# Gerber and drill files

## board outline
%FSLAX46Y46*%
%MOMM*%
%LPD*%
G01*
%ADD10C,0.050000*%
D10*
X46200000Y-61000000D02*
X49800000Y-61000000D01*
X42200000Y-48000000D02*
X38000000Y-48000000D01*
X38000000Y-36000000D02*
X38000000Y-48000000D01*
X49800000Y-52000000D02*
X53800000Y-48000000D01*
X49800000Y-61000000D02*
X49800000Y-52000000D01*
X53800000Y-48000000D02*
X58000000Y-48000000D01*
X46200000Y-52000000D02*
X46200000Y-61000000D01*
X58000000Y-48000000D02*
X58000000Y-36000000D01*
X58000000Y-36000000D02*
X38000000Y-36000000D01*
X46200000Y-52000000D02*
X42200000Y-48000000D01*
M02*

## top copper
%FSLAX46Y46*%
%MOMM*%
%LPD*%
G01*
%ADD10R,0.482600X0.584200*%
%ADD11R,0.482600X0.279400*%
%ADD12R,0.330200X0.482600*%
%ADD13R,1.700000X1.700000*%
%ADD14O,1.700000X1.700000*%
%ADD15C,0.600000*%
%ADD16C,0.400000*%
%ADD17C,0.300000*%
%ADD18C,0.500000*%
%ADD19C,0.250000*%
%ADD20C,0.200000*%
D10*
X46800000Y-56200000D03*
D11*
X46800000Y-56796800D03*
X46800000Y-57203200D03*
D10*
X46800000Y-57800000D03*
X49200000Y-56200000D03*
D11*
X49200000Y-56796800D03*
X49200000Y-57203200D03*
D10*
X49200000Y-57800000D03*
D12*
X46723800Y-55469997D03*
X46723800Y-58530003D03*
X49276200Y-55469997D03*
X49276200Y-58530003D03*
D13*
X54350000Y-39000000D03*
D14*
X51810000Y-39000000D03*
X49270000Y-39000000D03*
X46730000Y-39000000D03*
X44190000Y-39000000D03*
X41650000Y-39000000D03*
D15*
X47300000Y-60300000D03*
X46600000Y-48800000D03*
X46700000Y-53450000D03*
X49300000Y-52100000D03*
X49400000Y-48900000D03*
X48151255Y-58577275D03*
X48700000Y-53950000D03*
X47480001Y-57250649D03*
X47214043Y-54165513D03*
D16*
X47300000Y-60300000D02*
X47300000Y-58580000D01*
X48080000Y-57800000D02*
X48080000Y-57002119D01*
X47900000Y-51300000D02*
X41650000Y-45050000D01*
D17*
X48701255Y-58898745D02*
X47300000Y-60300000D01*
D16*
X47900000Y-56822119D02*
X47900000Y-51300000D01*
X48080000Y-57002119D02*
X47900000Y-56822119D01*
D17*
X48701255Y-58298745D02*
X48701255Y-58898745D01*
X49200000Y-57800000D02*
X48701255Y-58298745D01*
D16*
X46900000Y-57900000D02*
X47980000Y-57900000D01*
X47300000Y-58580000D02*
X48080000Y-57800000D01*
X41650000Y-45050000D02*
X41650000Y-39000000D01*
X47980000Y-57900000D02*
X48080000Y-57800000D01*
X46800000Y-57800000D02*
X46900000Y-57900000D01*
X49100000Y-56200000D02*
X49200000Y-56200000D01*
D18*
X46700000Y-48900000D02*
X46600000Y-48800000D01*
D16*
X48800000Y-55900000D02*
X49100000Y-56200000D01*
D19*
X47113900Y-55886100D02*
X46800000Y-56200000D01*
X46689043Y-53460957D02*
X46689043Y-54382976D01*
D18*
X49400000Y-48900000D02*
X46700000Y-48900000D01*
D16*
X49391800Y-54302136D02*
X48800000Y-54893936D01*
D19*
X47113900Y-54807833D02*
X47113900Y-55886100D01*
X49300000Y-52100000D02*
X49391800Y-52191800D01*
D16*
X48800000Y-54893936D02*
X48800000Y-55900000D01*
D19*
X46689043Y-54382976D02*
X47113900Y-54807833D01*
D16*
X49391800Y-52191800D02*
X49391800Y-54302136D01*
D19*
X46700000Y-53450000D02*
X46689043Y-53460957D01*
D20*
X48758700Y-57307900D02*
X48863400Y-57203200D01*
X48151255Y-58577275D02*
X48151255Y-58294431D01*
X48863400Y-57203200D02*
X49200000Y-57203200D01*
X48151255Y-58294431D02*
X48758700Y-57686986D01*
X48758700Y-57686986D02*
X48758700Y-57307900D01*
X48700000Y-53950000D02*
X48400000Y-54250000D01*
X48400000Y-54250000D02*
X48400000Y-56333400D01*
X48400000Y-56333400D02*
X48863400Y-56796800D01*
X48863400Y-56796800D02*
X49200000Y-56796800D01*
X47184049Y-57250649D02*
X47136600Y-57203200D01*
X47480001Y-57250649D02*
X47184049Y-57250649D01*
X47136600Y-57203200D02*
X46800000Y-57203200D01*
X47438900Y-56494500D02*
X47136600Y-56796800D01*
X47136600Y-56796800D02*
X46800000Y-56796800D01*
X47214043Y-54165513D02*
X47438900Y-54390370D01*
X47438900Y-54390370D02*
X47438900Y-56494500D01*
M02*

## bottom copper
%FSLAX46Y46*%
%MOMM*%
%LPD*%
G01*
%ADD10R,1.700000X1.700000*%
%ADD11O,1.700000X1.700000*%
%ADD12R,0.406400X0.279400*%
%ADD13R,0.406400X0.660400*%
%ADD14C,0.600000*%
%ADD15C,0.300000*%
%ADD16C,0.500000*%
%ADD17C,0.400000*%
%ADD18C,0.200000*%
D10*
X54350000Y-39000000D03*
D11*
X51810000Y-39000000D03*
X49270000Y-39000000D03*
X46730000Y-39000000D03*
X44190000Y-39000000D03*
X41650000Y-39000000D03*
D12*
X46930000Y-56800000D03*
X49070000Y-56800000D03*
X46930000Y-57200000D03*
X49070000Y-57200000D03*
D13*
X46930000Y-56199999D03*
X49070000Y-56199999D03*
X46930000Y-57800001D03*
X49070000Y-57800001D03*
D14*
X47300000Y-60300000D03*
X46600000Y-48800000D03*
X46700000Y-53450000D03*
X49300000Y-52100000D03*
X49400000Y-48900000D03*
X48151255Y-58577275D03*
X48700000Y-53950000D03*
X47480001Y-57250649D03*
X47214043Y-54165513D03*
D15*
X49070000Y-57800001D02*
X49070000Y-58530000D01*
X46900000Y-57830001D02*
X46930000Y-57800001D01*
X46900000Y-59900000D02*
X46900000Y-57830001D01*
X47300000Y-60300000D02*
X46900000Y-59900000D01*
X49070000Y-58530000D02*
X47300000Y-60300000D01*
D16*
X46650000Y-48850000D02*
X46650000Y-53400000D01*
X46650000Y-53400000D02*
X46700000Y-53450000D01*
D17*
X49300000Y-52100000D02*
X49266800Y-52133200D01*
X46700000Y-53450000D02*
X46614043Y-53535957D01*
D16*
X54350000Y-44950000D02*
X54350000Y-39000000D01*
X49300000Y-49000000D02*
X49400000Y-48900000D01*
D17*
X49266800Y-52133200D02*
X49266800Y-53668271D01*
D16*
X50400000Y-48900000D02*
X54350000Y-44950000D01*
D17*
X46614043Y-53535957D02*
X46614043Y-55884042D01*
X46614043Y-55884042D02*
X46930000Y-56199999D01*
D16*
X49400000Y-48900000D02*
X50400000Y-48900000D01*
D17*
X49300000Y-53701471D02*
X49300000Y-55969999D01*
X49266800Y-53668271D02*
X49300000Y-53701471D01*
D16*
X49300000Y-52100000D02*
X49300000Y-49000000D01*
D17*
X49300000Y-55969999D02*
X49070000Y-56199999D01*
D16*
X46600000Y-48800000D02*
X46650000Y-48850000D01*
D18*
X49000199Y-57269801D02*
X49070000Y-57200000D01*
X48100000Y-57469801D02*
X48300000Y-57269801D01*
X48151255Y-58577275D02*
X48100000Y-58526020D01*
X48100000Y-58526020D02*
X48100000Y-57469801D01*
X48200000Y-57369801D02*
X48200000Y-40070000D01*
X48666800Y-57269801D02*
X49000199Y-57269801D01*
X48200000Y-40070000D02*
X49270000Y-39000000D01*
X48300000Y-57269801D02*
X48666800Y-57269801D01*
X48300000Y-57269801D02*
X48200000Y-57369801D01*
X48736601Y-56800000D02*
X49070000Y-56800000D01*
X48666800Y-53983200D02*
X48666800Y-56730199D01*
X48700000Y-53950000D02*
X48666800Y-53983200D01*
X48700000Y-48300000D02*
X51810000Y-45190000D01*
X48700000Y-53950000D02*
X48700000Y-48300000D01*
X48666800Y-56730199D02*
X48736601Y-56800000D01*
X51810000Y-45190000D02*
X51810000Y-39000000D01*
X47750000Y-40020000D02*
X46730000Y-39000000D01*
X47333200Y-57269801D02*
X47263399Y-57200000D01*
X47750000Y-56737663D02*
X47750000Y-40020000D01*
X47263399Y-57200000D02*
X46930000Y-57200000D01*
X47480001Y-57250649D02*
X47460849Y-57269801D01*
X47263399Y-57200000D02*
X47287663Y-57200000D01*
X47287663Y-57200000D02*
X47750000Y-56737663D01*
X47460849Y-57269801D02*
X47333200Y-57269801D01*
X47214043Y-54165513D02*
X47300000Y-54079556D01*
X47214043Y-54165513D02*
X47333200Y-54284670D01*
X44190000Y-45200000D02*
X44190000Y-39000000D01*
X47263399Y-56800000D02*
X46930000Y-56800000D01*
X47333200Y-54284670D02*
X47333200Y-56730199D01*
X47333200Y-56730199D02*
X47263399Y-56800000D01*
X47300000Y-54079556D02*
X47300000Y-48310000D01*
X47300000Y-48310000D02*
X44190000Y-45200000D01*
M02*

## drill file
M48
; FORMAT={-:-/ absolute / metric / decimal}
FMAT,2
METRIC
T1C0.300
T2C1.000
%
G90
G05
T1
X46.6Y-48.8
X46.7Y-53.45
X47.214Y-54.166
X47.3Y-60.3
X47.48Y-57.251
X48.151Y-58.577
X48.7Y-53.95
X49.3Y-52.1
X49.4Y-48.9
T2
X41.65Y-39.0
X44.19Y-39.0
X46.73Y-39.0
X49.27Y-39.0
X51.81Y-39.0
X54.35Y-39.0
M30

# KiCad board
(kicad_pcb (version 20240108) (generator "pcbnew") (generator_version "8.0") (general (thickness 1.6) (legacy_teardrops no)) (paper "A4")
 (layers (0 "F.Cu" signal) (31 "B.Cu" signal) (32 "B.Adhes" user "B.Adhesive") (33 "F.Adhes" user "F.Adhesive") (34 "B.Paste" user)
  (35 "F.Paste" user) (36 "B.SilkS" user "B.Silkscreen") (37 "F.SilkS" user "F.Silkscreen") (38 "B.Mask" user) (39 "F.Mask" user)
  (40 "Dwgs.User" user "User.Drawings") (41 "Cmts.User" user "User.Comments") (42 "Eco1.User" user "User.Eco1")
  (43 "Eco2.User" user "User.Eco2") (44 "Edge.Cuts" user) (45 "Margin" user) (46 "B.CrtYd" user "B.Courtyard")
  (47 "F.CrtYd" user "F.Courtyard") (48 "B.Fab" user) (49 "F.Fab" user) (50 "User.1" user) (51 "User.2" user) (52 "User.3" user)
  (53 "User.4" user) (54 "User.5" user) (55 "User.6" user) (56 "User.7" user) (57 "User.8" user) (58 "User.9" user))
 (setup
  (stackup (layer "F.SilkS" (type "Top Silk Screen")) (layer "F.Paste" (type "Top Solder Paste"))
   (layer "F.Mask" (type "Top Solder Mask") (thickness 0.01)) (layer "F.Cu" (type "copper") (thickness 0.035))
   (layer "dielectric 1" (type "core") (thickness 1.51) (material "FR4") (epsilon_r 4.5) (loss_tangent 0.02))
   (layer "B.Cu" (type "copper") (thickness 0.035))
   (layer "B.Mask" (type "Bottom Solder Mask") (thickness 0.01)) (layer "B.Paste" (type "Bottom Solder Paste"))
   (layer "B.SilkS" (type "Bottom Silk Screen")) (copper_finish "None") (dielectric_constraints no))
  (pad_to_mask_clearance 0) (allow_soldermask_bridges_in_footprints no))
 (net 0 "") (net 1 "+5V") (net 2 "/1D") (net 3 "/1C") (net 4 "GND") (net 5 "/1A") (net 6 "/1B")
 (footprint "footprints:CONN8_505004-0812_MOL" (layer "F.Cu") (at 48 57 90)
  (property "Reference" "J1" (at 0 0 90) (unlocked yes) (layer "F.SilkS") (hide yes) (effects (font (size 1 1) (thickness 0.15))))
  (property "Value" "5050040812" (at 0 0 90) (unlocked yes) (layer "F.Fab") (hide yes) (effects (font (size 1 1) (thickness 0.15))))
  (pad "1" smd rect (at 0.8 -1.2 90) (size 0.5842 0.4826) (layers "F.Cu" "F.Paste" "F.Mask") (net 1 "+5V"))
  (pad "2" smd rect (at 0.2032 -1.2 90) (size 0.2794 0.4826) (layers "F.Cu" "F.Paste" "F.Mask") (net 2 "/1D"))
  (pad "3" smd rect (at -0.2032 -1.2 90) (size 0.2794 0.4826) (layers "F.Cu" "F.Paste" "F.Mask") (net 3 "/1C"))
  (pad "4" smd rect (at -0.8 -1.2 90) (size 0.5842 0.4826) (layers "F.Cu" "F.Paste" "F.Mask") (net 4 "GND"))
  (pad "5" smd rect (at 0.8 1.2 90) (size 0.5842 0.4826) (layers "F.Cu" "F.Paste" "F.Mask") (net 1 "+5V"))
  (pad "6" smd rect (at 0.2032 1.2 90) (size 0.2794 0.4826) (layers "F.Cu" "F.Paste" "F.Mask") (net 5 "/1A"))
  (pad "7" smd rect (at -0.2032 1.2 90) (size 0.2794 0.4826) (layers "F.Cu" "F.Paste" "F.Mask") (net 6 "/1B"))
  (pad "8" smd rect (at -0.8 1.2 90) (size 0.5842 0.4826) (layers "F.Cu" "F.Paste" "F.Mask") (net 4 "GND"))
  (pad "9" smd rect (at 1.530003 -1.2762 90) (size 0.4826 0.3302) (layers "F.Cu" "F.Paste" "F.Mask"))
  (pad "10" smd rect (at -1.530003 -1.2762 90) (size 0.4826 0.3302) (layers "F.Cu" "F.Paste" "F.Mask"))
  (pad "11" smd rect (at 1.530003 1.2762 90) (size 0.4826 0.3302) (layers "F.Cu" "F.Paste" "F.Mask"))
  (pad "12" smd rect (at -1.530003 1.2762 90) (size 0.4826 0.3302) (layers "F.Cu" "F.Paste" "F.Mask")))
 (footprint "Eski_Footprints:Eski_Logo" (layer "F.Cu") (at 48 47.65)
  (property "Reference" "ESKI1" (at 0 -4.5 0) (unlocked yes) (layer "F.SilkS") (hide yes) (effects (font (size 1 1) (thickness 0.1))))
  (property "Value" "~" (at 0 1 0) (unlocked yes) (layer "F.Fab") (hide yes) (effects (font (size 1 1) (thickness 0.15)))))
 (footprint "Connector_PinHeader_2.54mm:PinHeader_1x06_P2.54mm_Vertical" (layer "F.Cu") (at 54.35 39 -90)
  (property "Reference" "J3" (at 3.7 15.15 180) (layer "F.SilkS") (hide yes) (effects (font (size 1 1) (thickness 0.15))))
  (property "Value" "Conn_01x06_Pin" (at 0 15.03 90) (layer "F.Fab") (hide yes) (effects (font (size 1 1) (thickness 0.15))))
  (pad "1" thru_hole rect (at 0 0 270) (size 1.7 1.7) (drill 1) (layers "*.Cu" "*.Mask") (remove_unused_layers no) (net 1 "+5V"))
  (pad "2" thru_hole oval (at 0 2.54 270) (size 1.7 1.7) (drill 1) (layers "*.Cu" "*.Mask") (remove_unused_layers no) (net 5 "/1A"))
  (pad "3" thru_hole oval (at 0 5.08 270) (size 1.7 1.7) (drill 1) (layers "*.Cu" "*.Mask") (remove_unused_layers no) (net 6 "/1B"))
  (pad "4" thru_hole oval (at 0 7.62 270) (size 1.7 1.7) (drill 1) (layers "*.Cu" "*.Mask") (remove_unused_layers no) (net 3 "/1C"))
  (pad "5" thru_hole oval (at 0 10.16 270) (size 1.7 1.7) (drill 1) (layers "*.Cu" "*.Mask") (remove_unused_layers no) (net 2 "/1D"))
  (pad "6" thru_hole oval (at 0 12.7 270) (size 1.7 1.7) (drill 1) (layers "*.Cu" "*.Mask") (remove_unused_layers no) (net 4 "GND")))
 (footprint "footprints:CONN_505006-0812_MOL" (layer "B.Cu") (at 48 57 -90)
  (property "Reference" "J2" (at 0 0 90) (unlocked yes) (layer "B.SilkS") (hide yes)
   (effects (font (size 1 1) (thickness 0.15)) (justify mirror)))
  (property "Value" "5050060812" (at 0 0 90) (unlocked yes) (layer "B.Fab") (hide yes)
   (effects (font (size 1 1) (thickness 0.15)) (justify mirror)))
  (pad "1" smd rect (at -0.2 1.07 270) (size 0.2794 0.4064) (layers "B.Cu" "B.Paste" "B.Mask") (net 2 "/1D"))
  (pad "2" smd rect (at -0.2 -1.07 270) (size 0.2794 0.4064) (layers "B.Cu" "B.Paste" "B.Mask") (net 5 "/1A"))
  (pad "3" smd rect (at 0.2 1.07 270) (size 0.2794 0.4064) (layers "B.Cu" "B.Paste" "B.Mask") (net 3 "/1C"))
  (pad "4" smd rect (at 0.2 -1.07 270) (size 0.2794 0.4064) (layers "B.Cu" "B.Paste" "B.Mask") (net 6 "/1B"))
  (pad "P1" smd rect (at -0.800001 1.07 270) (size 0.6604 0.4064) (layers "B.Cu" "B.Paste" "B.Mask") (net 1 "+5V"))
  (pad "P2" smd rect (at -0.800001 -1.07 270) (size 0.6604 0.4064) (layers "B.Cu" "B.Paste" "B.Mask") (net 1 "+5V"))
  (pad "P3" smd rect (at 0.800001 1.07 270) (size 0.6604 0.4064) (layers "B.Cu" "B.Paste" "B.Mask") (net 4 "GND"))
  (pad "P4" smd rect (at 0.800001 -1.07 270) (size 0.6604 0.4064) (layers "B.Cu" "B.Paste" "B.Mask") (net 4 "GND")))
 (gr_line (start 46.2 61) (end 49.8 61) (stroke (width 0.05) (type default)) (layer "Edge.Cuts"))
 (gr_line (start 42.2 48) (end 38 48) (stroke (width 0.05) (type default)) (layer "Edge.Cuts"))
 (gr_line (start 38 36) (end 38 48) (stroke (width 0.05) (type default)) (layer "Edge.Cuts"))
 (gr_line (start 49.8 52) (end 53.8 48) (stroke (width 0.05) (type default)) (layer "Edge.Cuts"))
 (gr_line (start 49.8 61) (end 49.8 52) (stroke (width 0.05) (type default)) (layer "Edge.Cuts"))
 (gr_line (start 53.8 48) (end 58 48) (stroke (width 0.05) (type default)) (layer "Edge.Cuts"))
 (gr_line (start 46.2 52) (end 46.2 61) (stroke (width 0.05) (type default)) (layer "Edge.Cuts"))
 (gr_line (start 58 48) (end 58 36) (stroke (width 0.05) (type default)) (layer "Edge.Cuts"))
 (gr_line (start 58 36) (end 38 36) (stroke (width 0.05) (type default)) (layer "Edge.Cuts"))
 (gr_line (start 46.2 52) (end 42.2 48) (stroke (width 0.05) (type default)) (layer "Edge.Cuts"))
 (segment (start 47.3 60.3) (end 47.3 58.58) (width 0.4) (layer "F.Cu") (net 4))
 (segment (start 48.08 57.8) (end 48.08 57.002119) (width 0.4) (layer "F.Cu") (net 4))
 (segment (start 47.9 51.3) (end 41.65 45.05) (width 0.4) (layer "F.Cu") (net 4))
 (segment (start 48.701255 58.898745) (end 47.3 60.3) (width 0.3) (layer "F.Cu") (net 4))
 (segment (start 47.9 56.822119) (end 47.9 51.3) (width 0.4) (layer "F.Cu") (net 4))
 (segment (start 48.08 57.002119) (end 47.9 56.822119) (width 0.4) (layer "F.Cu") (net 4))
 (segment (start 48.701255 58.298745) (end 48.701255 58.898745) (width 0.3) (layer "F.Cu") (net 4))
 (segment (start 49.2 57.8) (end 48.701255 58.298745) (width 0.3) (layer "F.Cu") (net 4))
 (segment (start 46.9 57.9) (end 47.98 57.9) (width 0.4) (layer "F.Cu") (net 4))
 (segment (start 47.3 58.58) (end 48.08 57.8) (width 0.4) (layer "F.Cu") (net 4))
 (segment (start 41.65 45.05) (end 41.65 39) (width 0.4) (layer "F.Cu") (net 4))
 (segment (start 47.98 57.9) (end 48.08 57.8) (width 0.4) (layer "F.Cu") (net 4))
 (segment (start 46.8 57.8) (end 46.9 57.9) (width 0.4) (layer "F.Cu") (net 4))
 (via (at 47.3 60.3) (size 0.6) (drill 0.3) (layers "F.Cu" "B.Cu") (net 4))
 (segment (start 49.07 57.800001) (end 49.07 58.53) (width 0.3) (layer "B.Cu") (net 4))
 (segment (start 46.9 57.830001) (end 46.93 57.800001) (width 0.3) (layer "B.Cu") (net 4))
 (segment (start 46.9 59.9) (end 46.9 57.830001) (width 0.3) (layer "B.Cu") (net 4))
 (segment (start 47.3 60.3) (end 46.9 59.9) (width 0.3) (layer "B.Cu") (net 4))
 (segment (start 49.07 58.53) (end 47.3 60.3) (width 0.3) (layer "B.Cu") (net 4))
 (segment (start 49.1 56.2) (end 49.2 56.2) (width 0.4) (layer "F.Cu") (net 1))
 (segment (start 46.7 48.9) (end 46.6 48.8) (width 0.5) (layer "F.Cu") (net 1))
 (segment (start 48.8 55.9) (end 49.1 56.2) (width 0.4) (layer "F.Cu") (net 1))
 (segment (start 47.1139 55.8861) (end 46.8 56.2) (width 0.25) (layer "F.Cu") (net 1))
 (segment (start 46.689043 53.460957) (end 46.689043 54.382976) (width 0.25) (layer "F.Cu") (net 1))
 (segment (start 49.4 48.9) (end 46.7 48.9) (width 0.5) (layer "F.Cu") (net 1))
 (segment (start 49.3918 54.302136) (end 48.8 54.893936) (width 0.4) (layer "F.Cu") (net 1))
 (segment (start 47.1139 54.807833) (end 47.1139 55.8861) (width 0.25) (layer "F.Cu") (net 1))
 (segment (start 49.3 52.1) (end 49.3918 52.1918) (width 0.25) (layer "F.Cu") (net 1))
 (segment (start 48.8 54.893936) (end 48.8 55.9) (width 0.4) (layer "F.Cu") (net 1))
 (segment (start 46.689043 54.382976) (end 47.1139 54.807833) (width 0.25) (layer "F.Cu") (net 1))
 (segment (start 49.3918 52.1918) (end 49.3918 54.302136) (width 0.4) (layer "F.Cu") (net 1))
 (segment (start 46.7 53.45) (end 46.689043 53.460957) (width 0.25) (layer "F.Cu") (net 1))
 (via (at 46.6 48.8) (size 0.6) (drill 0.3) (layers "F.Cu" "B.Cu") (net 1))
 (via (at 46.7 53.45) (size 0.6) (drill 0.3) (layers "F.Cu" "B.Cu") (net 1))
 (via (at 49.3 52.1) (size 0.6) (drill 0.3) (layers "F.Cu" "B.Cu") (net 1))
 (via (at 49.4 48.9) (size 0.6) (drill 0.3) (layers "F.Cu" "B.Cu") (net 1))
 (segment (start 46.65 48.85) (end 46.65 53.4) (width 0.5) (layer "B.Cu") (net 1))
 (segment (start 46.65 53.4) (end 46.7 53.45) (width 0.5) (layer "B.Cu") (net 1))
 (segment (start 49.3 52.1) (end 49.2668 52.1332) (width 0.4) (layer "B.Cu") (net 1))
 (segment (start 46.7 53.45) (end 46.614043 53.535957) (width 0.4) (layer "B.Cu") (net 1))
 (segment (start 54.35 44.95) (end 54.35 39) (width 0.5) (layer "B.Cu") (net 1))
 (segment (start 49.3 49) (end 49.4 48.9) (width 0.5) (layer "B.Cu") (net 1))
 (segment (start 49.2668 52.1332) (end 49.2668 53.668271) (width 0.4) (layer "B.Cu") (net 1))
 (segment (start 50.4 48.9) (end 54.35 44.95) (width 0.5) (layer "B.Cu") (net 1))
 (segment (start 46.614043 53.535957) (end 46.614043 55.884042) (width 0.4) (layer "B.Cu") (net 1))
 (segment (start 46.614043 55.884042) (end 46.93 56.199999) (width 0.4) (layer "B.Cu") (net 1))
 (segment (start 49.4 48.9) (end 50.4 48.9) (width 0.5) (layer "B.Cu") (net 1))
 (segment (start 49.3 53.701471) (end 49.3 55.969999) (width 0.4) (layer "B.Cu") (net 1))
 (segment (start 49.2668 53.668271) (end 49.3 53.701471) (width 0.4) (layer "B.Cu") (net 1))
 (segment (start 49.3 52.1) (end 49.3 49) (width 0.5) (layer "B.Cu") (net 1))
 (segment (start 49.3 55.969999) (end 49.07 56.199999) (width 0.4) (layer "B.Cu") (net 1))
 (segment (start 46.6 48.8) (end 46.65 48.85) (width 0.5) (layer "B.Cu") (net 1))
 (segment (start 48.7587 57.3079) (end 48.8634 57.2032) (width 0.2) (layer "F.Cu") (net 6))
 (segment (start 48.151255 58.577275) (end 48.151255 58.294431) (width 0.2) (layer "F.Cu") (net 6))
 (segment (start 48.8634 57.2032) (end 49.2 57.2032) (width 0.2) (layer "F.Cu") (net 6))
 (segment (start 48.151255 58.294431) (end 48.7587 57.686986) (width 0.2) (layer "F.Cu") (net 6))
 (segment (start 48.7587 57.686986) (end 48.7587 57.3079) (width 0.2) (layer "F.Cu") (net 6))
 (via (at 48.151255 58.577275) (size 0.6) (drill 0.3) (layers "F.Cu" "B.Cu") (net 6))
 (segment (start 49.000199 57.269801) (end 49.07 57.2) (width 0.2) (layer "B.Cu") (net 6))
 (segment (start 48.1 57.469801) (end 48.3 57.269801) (width 0.2) (layer "B.Cu") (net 6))
 (segment (start 48.151255 58.577275) (end 48.1 58.52602) (width 0.2) (layer "B.Cu") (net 6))
 (segment (start 48.1 58.52602) (end 48.1 57.469801) (width 0.2) (layer "B.Cu") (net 6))
 (segment (start 48.2 57.369801) (end 48.2 40.07) (width 0.2) (layer "B.Cu") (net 6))
 (segment (start 48.6668 57.269801) (end 49.000199 57.269801) (width 0.2) (layer "B.Cu") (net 6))
 (segment (start 48.2 40.07) (end 49.27 39) (width 0.2) (layer "B.Cu") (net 6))
 (segment (start 48.3 57.269801) (end 48.6668 57.269801) (width 0.2) (layer "B.Cu") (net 6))
 (segment (start 48.3 57.269801) (end 48.2 57.369801) (width 0.2) (layer "B.Cu") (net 6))
 (segment (start 48.7 53.95) (end 48.4 54.25) (width 0.2) (layer "F.Cu") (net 5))
 (segment (start 48.4 54.25) (end 48.4 56.3334) (width 0.2) (layer "F.Cu") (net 5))
 (segment (start 48.4 56.3334) (end 48.8634 56.7968) (width 0.2) (layer "F.Cu") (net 5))
 (segment (start 48.8634 56.7968) (end 49.2 56.7968) (width 0.2) (layer "F.Cu") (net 5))
 (via (at 48.7 53.95) (size 0.6) (drill 0.3) (layers "F.Cu" "B.Cu") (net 5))
 (segment (start 48.736601 56.8) (end 49.07 56.8) (width 0.2) (layer "B.Cu") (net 5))
 (segment (start 48.6668 53.9832) (end 48.6668 56.730199) (width 0.2) (layer "B.Cu") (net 5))
 (segment (start 48.7 53.95) (end 48.6668 53.9832) (width 0.2) (layer "B.Cu") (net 5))
 (segment (start 48.7 48.3) (end 51.81 45.19) (width 0.2) (layer "B.Cu") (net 5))
 (segment (start 48.7 53.95) (end 48.7 48.3) (width 0.2) (layer "B.Cu") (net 5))
 (segment (start 48.6668 56.730199) (end 48.736601 56.8) (width 0.2) (layer "B.Cu") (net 5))
 (segment (start 51.81 45.19) (end 51.81 39) (width 0.2) (layer "B.Cu") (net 5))
 (segment (start 47.184049 57.250649) (end 47.1366 57.2032) (width 0.2) (layer "F.Cu") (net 3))
 (segment (start 47.480001 57.250649) (end 47.184049 57.250649) (width 0.2) (layer "F.Cu") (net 3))
 (segment (start 47.1366 57.2032) (end 46.8 57.2032) (width 0.2) (layer "F.Cu") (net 3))
 (via (at 47.480001 57.250649) (size 0.6) (drill 0.3) (layers "F.Cu" "B.Cu") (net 3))
 (segment (start 47.75 40.02) (end 46.73 39) (width 0.2) (layer "B.Cu") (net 3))
 (segment (start 47.3332 57.269801) (end 47.263399 57.2) (width 0.2) (layer "B.Cu") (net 3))
 (segment (start 47.75 56.737663) (end 47.75 40.02) (width 0.2) (layer "B.Cu") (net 3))
 (segment (start 47.263399 57.2) (end 46.93 57.2) (width 0.2) (layer "B.Cu") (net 3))
 (segment (start 47.480001 57.250649) (end 47.460849 57.269801) (width 0.2) (layer "B.Cu") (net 3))
 (segment (start 47.263399 57.2) (end 47.287663 57.2) (width 0.2) (layer "B.Cu") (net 3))
 (segment (start 47.287663 57.2) (end 47.75 56.737663) (width 0.2) (layer "B.Cu") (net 3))
 (segment (start 47.460849 57.269801) (end 47.3332 57.269801) (width 0.2) (layer "B.Cu") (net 3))
 (segment (start 47.4389 56.4945) (end 47.1366 56.7968) (width 0.2) (layer "F.Cu") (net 2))
 (segment (start 47.1366 56.7968) (end 46.8 56.7968) (width 0.2) (layer "F.Cu") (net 2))
 (segment (start 47.214043 54.165513) (end 47.4389 54.39037) (width 0.2) (layer "F.Cu") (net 2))
 (segment (start 47.4389 54.39037) (end 47.4389 56.4945) (width 0.2) (layer "F.Cu") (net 2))
 (via (at 47.214043 54.165513) (size 0.6) (drill 0.3) (layers "F.Cu" "B.Cu") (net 2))
 (segment (start 47.214043 54.165513) (end 47.3 54.079556) (width 0.2) (layer "B.Cu") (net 2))
 (segment (start 47.214043 54.165513) (end 47.3332 54.28467) (width 0.2) (layer "B.Cu") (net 2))
 (segment (start 44.19 45.2) (end 44.19 39) (width 0.2) (layer "B.Cu") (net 2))
 (segment (start 47.263399 56.8) (end 46.93 56.8) (width 0.2) (layer "B.Cu") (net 2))
 (segment (start 47.3332 54.28467) (end 47.3332 56.730199) (width 0.2) (layer "B.Cu") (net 2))
 (segment (start 47.3332 56.730199) (end 47.263399 56.8) (width 0.2) (layer "B.Cu") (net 2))
 (segment (start 47.3 54.079556) (end 47.3 48.31) (width 0.2) (layer "B.Cu") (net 2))
 (segment (start 47.3 48.31) (end 44.19 45.2) (width 0.2) (layer "B.Cu") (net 2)))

